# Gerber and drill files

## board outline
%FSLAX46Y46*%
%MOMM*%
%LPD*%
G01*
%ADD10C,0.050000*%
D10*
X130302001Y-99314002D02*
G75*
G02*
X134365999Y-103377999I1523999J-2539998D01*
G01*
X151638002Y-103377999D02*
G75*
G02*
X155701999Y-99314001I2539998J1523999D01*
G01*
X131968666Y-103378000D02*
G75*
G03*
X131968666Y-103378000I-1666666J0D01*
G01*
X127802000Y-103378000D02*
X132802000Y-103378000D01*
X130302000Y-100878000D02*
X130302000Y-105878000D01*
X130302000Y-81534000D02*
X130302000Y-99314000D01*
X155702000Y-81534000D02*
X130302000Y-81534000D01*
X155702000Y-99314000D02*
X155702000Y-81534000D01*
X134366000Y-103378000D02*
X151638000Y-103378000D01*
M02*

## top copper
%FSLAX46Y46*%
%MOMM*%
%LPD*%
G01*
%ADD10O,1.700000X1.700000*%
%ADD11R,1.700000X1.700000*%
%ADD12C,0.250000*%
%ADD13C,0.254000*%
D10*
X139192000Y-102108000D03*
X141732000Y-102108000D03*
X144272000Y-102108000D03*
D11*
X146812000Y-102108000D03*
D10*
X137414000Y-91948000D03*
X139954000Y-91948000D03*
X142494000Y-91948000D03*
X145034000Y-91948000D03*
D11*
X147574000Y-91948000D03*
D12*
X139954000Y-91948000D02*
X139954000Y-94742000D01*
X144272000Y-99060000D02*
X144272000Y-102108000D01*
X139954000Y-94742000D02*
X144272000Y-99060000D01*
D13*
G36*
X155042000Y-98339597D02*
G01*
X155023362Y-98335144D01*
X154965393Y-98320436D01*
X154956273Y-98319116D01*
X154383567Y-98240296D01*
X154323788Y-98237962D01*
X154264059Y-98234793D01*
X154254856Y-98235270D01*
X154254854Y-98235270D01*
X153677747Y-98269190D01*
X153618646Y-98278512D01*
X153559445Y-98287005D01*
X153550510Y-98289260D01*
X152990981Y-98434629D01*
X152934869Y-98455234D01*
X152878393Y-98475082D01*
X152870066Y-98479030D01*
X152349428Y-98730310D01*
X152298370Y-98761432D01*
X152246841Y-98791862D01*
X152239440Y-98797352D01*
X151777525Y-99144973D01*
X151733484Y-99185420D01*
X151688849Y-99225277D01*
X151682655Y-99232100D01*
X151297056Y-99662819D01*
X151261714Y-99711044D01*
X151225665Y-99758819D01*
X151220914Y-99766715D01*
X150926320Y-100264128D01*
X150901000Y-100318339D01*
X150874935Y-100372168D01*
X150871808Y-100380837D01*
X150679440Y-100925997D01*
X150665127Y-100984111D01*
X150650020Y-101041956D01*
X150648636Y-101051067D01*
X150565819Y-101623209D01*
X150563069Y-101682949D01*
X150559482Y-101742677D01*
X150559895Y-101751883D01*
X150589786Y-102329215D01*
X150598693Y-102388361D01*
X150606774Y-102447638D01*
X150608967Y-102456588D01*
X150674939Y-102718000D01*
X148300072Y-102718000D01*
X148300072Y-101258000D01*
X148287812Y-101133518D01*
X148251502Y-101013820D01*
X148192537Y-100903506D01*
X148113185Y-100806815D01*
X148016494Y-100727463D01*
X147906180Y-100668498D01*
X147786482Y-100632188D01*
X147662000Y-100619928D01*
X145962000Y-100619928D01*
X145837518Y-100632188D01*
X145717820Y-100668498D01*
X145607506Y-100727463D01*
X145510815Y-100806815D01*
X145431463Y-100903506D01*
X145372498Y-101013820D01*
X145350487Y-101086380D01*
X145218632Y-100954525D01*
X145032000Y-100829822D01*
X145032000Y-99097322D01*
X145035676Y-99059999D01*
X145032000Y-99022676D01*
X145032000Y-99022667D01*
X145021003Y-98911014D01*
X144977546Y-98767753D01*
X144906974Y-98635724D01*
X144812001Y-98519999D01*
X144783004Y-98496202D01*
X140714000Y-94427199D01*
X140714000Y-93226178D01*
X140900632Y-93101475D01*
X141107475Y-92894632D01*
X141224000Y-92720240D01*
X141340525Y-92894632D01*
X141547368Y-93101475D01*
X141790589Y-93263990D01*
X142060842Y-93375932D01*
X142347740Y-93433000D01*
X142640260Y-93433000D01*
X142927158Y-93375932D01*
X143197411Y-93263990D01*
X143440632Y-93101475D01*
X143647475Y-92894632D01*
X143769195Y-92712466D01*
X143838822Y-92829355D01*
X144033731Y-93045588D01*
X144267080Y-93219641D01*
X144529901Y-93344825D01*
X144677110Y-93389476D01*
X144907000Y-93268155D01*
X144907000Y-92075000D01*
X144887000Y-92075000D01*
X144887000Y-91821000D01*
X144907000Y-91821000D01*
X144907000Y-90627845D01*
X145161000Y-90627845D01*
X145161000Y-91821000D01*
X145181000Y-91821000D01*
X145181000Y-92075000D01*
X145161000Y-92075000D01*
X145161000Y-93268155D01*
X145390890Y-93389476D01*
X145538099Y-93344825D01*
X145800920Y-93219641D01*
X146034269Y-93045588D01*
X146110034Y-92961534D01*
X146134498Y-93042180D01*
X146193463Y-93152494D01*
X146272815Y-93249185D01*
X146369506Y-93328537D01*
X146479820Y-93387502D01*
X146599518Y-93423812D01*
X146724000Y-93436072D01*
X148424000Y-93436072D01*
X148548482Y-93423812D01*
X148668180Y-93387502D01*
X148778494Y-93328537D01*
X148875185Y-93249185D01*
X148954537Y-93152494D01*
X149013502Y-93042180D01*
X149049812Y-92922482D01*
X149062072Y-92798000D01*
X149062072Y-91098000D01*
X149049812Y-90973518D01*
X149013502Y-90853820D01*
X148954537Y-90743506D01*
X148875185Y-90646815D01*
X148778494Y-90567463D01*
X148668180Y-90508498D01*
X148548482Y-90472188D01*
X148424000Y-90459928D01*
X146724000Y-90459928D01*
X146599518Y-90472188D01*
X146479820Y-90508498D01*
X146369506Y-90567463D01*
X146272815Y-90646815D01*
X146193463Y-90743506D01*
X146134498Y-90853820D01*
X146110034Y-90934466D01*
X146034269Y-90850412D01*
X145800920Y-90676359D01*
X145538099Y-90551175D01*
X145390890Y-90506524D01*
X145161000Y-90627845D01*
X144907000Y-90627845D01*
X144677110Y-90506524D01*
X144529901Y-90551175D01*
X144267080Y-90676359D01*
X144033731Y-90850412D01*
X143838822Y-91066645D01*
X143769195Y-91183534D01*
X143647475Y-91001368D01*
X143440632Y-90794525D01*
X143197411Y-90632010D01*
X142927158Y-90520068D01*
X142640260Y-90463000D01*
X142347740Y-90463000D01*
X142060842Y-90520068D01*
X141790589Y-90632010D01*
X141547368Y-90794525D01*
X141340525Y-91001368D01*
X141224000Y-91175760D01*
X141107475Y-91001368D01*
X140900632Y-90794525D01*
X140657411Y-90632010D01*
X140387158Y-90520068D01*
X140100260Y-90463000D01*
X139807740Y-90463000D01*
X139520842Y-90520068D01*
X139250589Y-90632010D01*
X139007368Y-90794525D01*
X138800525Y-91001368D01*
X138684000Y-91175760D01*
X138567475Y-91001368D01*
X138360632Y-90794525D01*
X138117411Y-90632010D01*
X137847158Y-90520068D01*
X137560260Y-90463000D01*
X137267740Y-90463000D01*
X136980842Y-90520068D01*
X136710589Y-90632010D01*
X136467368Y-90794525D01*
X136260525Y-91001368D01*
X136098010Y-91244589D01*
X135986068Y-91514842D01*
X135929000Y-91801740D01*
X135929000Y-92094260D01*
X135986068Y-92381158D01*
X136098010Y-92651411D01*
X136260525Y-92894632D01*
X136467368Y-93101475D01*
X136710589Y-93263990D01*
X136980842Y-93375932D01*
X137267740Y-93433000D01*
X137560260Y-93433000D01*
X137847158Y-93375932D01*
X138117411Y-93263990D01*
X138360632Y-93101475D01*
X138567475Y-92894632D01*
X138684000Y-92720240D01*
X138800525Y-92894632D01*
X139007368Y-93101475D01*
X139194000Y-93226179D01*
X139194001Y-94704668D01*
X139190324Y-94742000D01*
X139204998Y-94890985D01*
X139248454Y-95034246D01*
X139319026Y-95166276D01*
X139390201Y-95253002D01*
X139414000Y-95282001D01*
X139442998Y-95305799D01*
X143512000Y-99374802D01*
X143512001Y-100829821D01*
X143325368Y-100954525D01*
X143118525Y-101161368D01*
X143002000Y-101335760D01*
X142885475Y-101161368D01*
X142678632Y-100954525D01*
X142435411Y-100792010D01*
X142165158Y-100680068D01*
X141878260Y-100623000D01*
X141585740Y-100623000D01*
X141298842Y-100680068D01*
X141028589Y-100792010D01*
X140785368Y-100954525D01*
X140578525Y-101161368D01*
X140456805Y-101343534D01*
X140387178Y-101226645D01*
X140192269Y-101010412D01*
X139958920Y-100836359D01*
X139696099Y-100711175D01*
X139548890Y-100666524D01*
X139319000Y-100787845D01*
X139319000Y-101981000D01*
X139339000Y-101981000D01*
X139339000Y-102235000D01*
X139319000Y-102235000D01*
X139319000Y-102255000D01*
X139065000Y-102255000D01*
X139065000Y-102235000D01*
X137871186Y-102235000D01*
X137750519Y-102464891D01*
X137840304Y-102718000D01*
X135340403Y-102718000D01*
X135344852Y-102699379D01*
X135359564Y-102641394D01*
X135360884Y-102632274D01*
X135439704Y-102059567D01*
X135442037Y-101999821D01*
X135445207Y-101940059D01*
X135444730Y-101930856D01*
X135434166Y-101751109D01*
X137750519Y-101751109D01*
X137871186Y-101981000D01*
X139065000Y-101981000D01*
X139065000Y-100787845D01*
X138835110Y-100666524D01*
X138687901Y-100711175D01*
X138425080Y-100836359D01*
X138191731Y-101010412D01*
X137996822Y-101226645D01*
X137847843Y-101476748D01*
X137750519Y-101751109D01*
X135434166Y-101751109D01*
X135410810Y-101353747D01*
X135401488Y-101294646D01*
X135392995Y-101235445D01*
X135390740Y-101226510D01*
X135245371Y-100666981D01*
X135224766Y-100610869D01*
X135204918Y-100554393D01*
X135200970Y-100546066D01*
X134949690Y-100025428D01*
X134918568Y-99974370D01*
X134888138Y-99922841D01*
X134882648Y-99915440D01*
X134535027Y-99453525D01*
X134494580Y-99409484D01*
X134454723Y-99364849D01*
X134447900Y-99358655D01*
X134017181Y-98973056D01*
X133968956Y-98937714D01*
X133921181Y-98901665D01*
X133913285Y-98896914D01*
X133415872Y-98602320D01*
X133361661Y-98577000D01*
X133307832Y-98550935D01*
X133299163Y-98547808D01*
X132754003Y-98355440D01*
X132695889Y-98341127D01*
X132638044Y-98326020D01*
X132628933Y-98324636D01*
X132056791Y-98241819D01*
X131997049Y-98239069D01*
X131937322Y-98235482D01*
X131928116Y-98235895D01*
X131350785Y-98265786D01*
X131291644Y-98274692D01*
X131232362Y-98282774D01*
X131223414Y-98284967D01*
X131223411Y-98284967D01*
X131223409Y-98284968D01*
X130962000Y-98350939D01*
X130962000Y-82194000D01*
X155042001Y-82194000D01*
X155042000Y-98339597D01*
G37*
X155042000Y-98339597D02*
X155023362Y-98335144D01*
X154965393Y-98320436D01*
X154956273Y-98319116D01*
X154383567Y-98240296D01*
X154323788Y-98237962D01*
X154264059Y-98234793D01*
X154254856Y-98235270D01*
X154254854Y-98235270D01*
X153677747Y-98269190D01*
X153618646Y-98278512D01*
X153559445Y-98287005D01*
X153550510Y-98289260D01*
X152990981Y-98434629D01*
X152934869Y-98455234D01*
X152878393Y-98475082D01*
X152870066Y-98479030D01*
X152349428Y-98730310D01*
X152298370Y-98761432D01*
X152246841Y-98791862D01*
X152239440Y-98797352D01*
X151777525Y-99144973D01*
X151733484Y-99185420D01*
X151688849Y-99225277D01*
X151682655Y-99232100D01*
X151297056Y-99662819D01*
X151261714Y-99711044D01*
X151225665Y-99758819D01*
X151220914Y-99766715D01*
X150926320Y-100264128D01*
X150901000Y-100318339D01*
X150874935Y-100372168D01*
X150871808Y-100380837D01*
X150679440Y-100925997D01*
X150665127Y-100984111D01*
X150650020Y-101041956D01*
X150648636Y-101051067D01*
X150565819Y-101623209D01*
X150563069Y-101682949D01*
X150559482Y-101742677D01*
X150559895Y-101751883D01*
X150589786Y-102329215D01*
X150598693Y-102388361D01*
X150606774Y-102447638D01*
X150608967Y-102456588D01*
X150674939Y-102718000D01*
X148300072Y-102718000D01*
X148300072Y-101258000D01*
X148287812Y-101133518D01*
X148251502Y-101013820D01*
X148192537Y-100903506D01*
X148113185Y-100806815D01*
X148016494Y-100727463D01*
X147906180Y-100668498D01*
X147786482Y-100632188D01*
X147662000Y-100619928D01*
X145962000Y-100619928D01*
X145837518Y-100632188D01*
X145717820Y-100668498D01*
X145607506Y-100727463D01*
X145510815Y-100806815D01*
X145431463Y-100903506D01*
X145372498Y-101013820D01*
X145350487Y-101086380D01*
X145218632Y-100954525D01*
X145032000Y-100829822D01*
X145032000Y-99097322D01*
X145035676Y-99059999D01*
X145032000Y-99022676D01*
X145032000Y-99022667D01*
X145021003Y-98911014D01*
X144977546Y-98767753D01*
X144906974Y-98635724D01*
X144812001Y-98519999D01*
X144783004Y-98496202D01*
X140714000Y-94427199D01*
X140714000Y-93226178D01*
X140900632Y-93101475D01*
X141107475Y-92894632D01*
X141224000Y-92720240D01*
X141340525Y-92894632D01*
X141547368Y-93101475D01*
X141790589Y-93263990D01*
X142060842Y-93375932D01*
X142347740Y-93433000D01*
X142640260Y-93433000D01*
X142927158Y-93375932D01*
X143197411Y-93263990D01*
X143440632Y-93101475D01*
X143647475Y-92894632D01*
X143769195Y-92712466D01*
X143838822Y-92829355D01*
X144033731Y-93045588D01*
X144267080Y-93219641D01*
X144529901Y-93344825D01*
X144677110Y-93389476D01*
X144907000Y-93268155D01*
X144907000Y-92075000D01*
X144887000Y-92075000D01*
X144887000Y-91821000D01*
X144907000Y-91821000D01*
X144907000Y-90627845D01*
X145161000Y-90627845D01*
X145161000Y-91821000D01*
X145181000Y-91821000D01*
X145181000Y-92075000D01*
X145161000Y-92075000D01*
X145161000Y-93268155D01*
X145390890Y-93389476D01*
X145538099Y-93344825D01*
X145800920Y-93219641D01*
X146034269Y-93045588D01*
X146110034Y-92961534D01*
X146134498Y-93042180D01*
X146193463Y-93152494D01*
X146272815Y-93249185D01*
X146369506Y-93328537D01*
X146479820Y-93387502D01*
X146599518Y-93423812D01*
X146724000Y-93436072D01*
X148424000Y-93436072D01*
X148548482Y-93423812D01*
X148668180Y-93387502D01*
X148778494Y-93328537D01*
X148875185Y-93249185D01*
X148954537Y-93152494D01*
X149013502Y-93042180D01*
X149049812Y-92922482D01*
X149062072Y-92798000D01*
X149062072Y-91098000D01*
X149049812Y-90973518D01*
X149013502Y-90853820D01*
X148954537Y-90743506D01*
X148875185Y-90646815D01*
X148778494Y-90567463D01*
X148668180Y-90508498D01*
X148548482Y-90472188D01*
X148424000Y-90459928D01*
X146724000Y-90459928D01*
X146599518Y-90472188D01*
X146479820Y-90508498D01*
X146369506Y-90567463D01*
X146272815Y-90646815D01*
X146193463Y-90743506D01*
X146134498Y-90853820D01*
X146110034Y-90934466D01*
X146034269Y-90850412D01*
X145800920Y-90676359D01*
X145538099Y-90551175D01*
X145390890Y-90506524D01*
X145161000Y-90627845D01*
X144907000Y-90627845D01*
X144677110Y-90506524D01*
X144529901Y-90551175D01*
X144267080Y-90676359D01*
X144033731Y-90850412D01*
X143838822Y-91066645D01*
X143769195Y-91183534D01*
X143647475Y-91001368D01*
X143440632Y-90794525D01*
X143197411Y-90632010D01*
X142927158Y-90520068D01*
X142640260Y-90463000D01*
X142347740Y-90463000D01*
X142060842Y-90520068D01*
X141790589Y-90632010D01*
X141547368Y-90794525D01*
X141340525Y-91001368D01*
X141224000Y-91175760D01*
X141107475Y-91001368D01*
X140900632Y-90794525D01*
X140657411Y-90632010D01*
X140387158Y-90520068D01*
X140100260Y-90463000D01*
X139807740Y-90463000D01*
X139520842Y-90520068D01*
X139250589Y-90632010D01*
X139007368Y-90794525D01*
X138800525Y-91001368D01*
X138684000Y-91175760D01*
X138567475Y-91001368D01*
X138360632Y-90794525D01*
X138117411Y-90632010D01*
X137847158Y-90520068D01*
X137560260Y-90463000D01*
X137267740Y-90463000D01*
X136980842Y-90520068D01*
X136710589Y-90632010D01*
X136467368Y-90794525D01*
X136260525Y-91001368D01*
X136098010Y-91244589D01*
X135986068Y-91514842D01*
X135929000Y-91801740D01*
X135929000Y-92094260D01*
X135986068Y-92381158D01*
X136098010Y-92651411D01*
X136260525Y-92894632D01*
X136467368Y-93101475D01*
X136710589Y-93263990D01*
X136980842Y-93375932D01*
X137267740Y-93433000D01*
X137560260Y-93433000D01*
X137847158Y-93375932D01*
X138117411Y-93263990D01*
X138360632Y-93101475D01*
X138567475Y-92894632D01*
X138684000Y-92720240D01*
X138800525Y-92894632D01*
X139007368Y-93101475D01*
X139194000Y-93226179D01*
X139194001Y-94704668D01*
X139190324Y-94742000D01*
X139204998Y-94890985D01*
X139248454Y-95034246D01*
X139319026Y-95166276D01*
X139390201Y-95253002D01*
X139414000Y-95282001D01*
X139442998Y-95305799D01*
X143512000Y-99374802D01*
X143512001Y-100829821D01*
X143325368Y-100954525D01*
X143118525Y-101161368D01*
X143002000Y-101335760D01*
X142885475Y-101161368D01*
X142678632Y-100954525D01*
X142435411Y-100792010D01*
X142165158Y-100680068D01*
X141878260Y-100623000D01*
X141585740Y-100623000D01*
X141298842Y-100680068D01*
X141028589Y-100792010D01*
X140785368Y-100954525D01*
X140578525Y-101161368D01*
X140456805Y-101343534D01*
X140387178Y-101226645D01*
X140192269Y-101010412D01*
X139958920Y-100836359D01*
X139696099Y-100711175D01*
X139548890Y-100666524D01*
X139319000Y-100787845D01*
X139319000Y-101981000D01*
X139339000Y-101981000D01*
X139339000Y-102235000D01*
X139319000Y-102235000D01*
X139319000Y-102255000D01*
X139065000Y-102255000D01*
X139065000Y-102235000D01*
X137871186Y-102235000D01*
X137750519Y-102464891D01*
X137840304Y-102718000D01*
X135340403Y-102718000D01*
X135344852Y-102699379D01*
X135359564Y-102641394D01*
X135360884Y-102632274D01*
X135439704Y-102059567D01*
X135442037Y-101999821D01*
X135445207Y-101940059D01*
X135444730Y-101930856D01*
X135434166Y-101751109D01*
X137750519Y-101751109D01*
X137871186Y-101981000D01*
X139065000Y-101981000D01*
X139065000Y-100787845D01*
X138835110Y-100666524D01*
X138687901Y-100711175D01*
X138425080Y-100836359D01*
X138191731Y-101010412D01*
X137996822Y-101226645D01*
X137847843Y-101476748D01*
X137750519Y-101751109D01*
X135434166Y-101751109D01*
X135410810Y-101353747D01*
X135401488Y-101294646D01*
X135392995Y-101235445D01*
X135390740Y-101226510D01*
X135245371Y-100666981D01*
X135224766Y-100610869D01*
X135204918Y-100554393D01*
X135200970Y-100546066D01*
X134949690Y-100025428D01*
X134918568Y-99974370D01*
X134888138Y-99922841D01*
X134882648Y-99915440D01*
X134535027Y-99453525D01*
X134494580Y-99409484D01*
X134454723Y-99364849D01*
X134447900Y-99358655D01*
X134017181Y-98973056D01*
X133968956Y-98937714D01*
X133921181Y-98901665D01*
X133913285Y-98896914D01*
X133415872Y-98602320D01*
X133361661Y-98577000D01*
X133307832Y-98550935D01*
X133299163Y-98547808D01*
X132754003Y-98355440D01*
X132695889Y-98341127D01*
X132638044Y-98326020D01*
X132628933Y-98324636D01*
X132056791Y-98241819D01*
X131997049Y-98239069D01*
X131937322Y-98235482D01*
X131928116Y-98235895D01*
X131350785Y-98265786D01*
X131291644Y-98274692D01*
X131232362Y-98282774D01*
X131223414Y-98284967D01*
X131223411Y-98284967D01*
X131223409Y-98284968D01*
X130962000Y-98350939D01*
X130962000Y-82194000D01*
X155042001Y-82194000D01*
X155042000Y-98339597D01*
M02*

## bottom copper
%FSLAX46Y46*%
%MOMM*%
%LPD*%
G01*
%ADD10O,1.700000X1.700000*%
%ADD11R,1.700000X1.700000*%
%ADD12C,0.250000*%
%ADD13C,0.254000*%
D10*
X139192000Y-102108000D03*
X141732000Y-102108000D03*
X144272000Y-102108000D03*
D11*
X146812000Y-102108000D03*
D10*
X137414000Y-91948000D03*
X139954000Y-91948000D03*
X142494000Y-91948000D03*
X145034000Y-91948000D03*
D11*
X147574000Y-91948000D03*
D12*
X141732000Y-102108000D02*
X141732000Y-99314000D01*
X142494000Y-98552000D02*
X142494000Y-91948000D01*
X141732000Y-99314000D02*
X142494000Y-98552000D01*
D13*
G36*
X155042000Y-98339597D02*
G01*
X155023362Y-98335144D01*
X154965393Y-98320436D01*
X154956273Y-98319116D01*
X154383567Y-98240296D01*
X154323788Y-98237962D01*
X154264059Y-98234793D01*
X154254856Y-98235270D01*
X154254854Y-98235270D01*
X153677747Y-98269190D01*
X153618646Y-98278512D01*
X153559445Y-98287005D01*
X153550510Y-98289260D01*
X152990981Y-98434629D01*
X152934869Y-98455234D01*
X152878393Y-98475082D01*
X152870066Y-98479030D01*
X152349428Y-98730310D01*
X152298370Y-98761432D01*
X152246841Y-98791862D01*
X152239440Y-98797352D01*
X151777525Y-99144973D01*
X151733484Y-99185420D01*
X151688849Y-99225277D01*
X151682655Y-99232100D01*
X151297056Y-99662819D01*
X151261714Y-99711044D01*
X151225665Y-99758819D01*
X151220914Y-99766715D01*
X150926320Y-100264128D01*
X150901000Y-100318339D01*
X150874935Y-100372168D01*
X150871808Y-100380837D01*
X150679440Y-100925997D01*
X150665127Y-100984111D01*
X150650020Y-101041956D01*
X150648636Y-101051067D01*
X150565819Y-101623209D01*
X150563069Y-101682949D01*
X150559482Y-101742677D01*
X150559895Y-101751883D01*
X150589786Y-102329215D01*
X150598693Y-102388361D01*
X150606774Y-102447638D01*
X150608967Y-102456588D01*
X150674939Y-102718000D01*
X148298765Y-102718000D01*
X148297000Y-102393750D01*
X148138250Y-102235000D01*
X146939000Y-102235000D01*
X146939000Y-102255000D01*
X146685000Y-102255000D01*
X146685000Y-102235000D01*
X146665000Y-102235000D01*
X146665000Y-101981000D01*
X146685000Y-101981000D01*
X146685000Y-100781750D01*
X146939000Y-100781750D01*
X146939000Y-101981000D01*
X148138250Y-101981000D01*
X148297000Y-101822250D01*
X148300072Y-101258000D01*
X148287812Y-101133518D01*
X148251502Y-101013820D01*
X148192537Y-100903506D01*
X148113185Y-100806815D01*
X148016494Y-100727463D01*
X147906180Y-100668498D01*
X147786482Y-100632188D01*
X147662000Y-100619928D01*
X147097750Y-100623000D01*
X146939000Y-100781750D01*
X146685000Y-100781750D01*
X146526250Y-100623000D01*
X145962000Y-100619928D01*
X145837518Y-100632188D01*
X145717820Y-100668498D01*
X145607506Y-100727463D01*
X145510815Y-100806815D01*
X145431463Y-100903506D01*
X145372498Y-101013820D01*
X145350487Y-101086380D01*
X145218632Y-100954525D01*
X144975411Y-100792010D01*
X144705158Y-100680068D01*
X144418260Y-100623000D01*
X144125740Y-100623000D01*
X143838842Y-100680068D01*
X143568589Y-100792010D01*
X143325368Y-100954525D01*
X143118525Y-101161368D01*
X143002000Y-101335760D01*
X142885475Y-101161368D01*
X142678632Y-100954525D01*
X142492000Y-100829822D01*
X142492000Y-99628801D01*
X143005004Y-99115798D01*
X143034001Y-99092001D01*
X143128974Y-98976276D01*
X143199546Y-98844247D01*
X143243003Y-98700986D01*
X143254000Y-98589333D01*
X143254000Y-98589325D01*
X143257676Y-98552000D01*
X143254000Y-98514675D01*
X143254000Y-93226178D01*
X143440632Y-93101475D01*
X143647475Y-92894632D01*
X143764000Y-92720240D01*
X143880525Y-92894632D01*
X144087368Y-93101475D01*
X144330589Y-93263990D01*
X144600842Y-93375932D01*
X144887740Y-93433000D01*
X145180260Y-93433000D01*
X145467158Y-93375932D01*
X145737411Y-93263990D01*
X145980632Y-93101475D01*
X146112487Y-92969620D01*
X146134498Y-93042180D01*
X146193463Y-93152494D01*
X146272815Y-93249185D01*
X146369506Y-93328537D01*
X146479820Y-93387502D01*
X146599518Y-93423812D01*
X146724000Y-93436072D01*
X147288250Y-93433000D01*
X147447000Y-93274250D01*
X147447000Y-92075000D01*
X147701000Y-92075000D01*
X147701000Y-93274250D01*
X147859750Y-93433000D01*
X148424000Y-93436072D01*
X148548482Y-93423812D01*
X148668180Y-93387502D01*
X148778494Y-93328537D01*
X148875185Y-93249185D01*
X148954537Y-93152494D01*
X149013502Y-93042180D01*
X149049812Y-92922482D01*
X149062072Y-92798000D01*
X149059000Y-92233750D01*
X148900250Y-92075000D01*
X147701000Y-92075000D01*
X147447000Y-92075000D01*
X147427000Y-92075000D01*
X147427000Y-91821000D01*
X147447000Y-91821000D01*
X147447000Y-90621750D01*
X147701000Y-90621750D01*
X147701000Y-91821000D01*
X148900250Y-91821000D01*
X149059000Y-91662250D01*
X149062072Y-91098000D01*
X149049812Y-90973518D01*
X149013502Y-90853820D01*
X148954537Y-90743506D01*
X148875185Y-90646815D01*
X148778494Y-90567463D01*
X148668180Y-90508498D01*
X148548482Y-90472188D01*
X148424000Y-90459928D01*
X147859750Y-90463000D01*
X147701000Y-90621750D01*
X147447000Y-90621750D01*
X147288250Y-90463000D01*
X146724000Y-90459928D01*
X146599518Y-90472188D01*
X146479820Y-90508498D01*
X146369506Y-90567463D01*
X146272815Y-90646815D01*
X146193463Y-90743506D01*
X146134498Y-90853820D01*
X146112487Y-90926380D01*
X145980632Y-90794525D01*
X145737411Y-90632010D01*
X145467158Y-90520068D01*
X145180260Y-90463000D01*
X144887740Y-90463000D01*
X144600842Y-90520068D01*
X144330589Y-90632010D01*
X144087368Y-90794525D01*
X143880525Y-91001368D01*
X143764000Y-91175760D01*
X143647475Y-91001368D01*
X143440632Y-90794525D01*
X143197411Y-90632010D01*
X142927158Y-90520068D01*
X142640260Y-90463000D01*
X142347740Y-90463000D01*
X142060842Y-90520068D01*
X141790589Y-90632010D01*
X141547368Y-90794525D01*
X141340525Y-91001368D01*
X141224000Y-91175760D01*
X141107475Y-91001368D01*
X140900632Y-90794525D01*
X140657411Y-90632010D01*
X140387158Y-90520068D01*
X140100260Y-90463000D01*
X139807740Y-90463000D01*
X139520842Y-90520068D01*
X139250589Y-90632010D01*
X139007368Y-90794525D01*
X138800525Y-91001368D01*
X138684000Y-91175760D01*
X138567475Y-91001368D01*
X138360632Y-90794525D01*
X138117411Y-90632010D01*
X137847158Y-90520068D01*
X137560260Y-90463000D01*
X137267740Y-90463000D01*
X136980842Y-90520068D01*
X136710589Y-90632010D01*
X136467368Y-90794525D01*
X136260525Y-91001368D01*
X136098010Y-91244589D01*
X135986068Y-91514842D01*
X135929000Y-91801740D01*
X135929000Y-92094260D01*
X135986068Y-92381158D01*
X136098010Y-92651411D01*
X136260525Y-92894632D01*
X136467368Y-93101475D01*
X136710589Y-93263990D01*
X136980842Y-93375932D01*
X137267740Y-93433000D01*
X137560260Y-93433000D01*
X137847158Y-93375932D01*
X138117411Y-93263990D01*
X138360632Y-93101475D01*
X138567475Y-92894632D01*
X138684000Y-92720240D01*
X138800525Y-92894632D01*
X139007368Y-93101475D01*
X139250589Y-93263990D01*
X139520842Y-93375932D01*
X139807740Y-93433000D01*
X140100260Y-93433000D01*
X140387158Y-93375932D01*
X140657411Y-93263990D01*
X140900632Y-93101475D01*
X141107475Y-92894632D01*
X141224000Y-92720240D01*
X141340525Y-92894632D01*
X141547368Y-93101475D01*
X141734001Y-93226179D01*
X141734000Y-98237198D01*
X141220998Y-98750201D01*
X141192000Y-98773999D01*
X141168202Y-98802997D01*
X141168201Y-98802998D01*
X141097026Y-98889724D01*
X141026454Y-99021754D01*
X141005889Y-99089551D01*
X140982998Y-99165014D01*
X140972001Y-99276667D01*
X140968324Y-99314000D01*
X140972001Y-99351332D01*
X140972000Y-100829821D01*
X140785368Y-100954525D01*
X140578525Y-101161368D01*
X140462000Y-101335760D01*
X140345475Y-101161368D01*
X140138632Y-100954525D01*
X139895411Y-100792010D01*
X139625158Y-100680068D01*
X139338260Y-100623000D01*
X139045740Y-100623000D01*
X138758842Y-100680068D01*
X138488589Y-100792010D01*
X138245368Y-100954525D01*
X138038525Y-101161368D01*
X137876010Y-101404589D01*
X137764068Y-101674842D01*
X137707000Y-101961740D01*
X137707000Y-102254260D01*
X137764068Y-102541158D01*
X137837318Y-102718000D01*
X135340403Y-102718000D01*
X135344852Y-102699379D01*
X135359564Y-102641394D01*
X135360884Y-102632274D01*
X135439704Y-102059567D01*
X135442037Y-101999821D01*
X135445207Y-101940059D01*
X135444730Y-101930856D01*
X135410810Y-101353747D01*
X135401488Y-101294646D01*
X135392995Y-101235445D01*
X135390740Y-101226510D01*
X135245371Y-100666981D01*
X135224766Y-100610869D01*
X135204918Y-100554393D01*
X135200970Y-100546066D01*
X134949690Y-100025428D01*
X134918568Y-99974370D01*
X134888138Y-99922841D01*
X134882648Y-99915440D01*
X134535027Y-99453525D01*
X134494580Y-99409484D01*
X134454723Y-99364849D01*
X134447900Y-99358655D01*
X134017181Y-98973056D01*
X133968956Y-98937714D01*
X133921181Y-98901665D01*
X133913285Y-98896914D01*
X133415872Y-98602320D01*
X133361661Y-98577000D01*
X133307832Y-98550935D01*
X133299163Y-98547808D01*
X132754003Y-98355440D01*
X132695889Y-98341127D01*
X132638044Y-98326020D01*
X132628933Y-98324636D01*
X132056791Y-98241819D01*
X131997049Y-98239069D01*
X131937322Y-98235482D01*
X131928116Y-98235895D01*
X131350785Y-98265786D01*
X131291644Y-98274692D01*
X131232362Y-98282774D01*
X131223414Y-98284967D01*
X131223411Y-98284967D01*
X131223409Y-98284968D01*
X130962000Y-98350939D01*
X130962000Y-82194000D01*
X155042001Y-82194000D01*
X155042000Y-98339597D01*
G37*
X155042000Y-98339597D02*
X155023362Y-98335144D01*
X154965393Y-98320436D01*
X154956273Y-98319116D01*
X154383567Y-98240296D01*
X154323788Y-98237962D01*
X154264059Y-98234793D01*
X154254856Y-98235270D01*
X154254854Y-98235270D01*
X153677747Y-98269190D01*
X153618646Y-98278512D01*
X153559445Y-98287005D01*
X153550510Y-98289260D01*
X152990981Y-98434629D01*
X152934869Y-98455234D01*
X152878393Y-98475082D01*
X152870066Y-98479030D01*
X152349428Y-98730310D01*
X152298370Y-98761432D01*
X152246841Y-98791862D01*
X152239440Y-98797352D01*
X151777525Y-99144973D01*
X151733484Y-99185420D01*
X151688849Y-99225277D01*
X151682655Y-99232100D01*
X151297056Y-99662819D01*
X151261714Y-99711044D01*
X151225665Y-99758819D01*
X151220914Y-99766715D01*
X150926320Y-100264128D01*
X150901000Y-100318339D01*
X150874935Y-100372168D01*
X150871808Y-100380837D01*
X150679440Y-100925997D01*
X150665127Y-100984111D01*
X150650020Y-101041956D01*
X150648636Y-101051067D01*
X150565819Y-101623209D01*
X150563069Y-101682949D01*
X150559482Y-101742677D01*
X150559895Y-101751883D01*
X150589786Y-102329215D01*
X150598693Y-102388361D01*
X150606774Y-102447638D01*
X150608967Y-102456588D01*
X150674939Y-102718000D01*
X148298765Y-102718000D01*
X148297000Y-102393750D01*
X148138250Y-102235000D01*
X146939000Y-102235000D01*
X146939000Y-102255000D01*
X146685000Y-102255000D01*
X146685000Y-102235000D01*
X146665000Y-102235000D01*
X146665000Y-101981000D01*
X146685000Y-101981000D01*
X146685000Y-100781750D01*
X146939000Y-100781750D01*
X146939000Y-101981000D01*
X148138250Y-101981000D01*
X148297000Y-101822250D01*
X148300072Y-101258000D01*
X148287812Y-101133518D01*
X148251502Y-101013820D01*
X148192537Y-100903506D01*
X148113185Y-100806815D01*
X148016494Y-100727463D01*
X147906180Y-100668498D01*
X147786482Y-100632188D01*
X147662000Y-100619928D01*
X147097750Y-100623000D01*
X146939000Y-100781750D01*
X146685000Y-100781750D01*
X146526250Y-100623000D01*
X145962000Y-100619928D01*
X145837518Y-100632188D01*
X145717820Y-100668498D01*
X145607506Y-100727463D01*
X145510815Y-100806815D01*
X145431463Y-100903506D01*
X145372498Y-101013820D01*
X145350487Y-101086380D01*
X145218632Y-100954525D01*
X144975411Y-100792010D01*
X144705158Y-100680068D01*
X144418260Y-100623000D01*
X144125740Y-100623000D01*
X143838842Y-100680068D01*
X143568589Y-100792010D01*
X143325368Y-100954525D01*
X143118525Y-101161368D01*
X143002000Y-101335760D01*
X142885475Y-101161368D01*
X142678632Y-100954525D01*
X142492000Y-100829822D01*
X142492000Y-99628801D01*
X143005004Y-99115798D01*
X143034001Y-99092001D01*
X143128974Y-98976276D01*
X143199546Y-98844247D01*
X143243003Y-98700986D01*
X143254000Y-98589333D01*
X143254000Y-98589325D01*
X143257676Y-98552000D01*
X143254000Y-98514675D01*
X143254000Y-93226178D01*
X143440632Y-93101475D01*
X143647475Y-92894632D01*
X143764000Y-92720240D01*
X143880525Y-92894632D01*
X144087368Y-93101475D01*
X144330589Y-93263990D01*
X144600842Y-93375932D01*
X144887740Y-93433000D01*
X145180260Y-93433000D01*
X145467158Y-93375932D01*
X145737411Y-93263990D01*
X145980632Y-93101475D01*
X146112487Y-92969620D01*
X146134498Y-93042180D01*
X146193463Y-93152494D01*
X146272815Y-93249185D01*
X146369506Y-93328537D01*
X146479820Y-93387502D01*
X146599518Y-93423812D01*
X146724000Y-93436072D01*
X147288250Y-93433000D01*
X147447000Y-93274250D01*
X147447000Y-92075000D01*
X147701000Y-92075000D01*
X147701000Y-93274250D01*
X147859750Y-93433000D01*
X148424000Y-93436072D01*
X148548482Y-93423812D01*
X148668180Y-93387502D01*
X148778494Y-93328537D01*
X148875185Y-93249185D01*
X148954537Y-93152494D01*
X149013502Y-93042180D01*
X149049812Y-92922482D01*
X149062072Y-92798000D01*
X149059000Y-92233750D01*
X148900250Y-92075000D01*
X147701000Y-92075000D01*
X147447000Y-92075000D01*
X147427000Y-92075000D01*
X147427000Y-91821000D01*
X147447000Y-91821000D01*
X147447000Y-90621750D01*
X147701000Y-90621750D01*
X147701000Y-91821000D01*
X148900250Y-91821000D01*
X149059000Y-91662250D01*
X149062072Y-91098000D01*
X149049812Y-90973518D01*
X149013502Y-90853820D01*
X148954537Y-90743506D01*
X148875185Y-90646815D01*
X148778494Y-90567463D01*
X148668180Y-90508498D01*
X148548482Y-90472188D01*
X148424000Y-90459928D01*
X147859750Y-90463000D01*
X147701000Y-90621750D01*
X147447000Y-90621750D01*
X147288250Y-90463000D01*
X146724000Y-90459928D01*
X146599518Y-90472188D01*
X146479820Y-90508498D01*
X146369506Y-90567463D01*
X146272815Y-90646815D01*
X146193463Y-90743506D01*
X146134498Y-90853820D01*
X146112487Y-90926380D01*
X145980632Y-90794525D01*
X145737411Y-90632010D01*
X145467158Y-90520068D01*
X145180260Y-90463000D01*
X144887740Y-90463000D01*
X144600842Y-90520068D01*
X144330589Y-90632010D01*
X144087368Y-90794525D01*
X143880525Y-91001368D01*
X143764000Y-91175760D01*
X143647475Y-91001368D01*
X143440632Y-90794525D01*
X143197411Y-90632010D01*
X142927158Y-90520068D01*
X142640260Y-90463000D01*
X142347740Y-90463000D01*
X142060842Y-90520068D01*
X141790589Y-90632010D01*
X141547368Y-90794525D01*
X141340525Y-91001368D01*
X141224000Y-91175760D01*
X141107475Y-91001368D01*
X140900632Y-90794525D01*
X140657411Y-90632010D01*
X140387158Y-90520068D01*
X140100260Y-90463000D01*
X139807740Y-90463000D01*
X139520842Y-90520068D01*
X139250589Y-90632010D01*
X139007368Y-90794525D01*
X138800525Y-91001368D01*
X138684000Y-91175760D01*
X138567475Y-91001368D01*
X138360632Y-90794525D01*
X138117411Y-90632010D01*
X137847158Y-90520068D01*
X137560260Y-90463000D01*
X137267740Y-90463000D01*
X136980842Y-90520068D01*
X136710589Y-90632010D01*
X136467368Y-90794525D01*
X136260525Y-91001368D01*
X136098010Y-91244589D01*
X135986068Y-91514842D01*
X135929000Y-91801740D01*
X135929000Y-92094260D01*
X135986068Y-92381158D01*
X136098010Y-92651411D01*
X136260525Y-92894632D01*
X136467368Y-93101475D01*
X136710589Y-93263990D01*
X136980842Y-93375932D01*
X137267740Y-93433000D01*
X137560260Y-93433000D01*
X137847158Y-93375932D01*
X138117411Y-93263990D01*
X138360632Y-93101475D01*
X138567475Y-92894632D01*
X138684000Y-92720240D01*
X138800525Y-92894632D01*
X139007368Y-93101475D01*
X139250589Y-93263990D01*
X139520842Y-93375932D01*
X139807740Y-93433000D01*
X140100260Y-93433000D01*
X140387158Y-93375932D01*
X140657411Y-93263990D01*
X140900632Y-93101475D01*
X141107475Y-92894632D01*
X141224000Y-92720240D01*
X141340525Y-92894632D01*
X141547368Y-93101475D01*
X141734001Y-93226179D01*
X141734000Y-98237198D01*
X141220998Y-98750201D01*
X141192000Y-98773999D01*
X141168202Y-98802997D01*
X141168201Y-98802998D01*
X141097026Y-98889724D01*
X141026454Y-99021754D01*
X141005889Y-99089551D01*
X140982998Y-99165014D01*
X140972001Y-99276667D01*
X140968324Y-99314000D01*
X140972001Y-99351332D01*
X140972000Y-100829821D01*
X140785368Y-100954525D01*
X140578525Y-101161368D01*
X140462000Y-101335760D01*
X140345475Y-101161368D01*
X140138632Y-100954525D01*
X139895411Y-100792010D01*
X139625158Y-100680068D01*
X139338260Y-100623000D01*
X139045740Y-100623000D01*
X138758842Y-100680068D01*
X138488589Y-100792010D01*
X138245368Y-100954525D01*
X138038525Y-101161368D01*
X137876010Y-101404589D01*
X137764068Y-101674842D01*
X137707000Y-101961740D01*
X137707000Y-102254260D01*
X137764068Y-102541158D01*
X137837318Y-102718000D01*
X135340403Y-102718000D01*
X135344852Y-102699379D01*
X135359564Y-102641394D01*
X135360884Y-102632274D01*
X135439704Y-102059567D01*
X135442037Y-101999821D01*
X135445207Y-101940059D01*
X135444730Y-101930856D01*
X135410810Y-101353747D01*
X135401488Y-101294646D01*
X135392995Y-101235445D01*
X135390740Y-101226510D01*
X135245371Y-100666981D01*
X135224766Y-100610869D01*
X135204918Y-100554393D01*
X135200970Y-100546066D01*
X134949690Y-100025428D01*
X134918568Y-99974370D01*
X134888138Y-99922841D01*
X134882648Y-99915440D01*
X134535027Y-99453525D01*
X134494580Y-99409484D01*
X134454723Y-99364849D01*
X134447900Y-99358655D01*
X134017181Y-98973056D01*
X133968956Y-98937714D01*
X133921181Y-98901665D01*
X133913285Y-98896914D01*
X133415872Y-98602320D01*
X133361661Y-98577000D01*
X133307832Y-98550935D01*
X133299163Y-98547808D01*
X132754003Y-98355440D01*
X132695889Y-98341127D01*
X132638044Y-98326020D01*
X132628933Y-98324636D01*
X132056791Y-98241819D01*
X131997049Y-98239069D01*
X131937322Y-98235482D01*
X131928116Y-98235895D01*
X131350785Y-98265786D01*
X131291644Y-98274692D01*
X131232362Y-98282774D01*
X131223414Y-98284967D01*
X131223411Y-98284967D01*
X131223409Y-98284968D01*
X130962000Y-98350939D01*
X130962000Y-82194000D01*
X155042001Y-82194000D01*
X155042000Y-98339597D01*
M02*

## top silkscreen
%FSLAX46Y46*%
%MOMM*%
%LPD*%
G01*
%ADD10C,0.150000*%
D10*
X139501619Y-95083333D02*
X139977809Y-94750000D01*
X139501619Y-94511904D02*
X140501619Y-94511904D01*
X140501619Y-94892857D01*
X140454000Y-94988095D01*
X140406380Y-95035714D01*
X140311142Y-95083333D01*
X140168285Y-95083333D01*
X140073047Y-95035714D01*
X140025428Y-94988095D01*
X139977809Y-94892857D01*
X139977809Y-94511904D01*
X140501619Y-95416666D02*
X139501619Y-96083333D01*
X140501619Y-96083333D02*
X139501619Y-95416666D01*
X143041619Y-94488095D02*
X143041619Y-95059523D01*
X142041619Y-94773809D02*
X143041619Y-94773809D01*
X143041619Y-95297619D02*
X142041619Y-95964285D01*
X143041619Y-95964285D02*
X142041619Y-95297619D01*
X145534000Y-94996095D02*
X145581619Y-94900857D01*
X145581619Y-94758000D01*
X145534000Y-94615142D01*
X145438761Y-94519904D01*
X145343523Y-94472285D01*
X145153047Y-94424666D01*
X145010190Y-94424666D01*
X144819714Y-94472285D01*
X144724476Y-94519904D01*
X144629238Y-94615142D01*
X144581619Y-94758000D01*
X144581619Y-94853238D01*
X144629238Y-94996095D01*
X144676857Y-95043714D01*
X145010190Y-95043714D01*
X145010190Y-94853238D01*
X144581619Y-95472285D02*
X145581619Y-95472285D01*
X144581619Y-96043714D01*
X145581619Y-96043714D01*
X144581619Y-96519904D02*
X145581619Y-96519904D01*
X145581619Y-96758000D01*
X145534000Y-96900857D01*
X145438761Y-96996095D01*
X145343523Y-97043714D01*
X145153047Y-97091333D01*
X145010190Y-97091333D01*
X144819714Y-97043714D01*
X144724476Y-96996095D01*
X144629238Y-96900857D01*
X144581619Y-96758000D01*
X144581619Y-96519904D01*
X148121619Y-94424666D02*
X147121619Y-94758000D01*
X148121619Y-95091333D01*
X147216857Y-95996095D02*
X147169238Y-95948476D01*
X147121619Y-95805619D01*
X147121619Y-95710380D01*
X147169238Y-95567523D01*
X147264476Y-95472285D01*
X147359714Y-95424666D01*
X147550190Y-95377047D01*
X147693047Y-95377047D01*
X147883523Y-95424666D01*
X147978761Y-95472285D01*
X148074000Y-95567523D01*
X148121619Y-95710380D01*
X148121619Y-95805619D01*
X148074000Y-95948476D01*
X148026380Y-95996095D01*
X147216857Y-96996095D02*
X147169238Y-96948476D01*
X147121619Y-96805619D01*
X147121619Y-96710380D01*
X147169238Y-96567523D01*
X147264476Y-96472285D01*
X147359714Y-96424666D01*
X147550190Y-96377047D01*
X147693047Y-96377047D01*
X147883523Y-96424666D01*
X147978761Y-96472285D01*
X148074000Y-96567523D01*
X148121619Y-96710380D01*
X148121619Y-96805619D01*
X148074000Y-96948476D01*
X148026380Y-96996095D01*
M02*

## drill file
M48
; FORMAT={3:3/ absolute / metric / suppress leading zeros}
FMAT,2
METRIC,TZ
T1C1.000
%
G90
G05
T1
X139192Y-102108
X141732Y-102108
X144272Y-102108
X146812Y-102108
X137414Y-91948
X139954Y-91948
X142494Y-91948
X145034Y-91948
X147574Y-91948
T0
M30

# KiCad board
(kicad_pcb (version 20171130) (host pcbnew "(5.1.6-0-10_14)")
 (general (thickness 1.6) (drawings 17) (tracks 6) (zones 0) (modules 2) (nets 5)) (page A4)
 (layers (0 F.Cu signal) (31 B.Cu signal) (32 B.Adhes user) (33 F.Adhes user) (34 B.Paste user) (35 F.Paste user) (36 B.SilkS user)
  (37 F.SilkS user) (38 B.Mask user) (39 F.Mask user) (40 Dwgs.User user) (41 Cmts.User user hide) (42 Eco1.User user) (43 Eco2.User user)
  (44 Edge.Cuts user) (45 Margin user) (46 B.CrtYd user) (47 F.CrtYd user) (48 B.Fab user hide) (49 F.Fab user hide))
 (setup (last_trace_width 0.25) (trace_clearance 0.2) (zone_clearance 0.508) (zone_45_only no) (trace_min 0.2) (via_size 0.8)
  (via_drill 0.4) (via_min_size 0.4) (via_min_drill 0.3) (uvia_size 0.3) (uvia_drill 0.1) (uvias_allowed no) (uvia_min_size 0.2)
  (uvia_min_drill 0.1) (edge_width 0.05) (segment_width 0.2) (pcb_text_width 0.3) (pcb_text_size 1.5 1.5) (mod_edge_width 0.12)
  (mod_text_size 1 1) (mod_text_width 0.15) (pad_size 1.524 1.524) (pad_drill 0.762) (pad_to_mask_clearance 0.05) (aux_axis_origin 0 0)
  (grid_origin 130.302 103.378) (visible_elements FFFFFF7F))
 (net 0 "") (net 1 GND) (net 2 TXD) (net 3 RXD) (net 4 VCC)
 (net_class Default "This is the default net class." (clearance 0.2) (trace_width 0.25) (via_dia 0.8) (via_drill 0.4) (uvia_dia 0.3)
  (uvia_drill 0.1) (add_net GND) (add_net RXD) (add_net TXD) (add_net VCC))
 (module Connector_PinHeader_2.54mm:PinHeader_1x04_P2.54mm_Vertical (layer B.Cu) (at 146.812 102.108 90)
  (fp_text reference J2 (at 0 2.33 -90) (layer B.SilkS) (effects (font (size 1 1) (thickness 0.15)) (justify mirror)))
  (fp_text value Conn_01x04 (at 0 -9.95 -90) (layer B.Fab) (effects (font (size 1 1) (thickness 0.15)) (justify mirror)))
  (pad 4 thru_hole oval (at 0 -7.62 90) (size 1.7 1.7) (drill 1) (layers *.Cu *.Mask) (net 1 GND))
  (pad 3 thru_hole oval (at 0 -5.08 90) (size 1.7 1.7) (drill 1) (layers *.Cu *.Mask) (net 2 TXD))
  (pad 2 thru_hole oval (at 0 -2.54 90) (size 1.7 1.7) (drill 1) (layers *.Cu *.Mask) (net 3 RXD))
  (pad 1 thru_hole rect (at 0 0 90) (size 1.7 1.7) (drill 1) (layers *.Cu *.Mask) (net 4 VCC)))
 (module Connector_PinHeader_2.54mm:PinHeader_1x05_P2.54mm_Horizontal (layer B.Cu) (at 147.574 91.948 90)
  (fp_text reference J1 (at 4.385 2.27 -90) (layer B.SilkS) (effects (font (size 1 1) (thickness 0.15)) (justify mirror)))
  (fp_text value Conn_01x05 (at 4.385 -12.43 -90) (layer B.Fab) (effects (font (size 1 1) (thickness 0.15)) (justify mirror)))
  (pad 5 thru_hole oval (at 0 -10.16 90) (size 1.7 1.7) (drill 1) (layers *.Cu *.Mask))
  (pad 4 thru_hole oval (at 0 -7.62 90) (size 1.7 1.7) (drill 1) (layers *.Cu *.Mask) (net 3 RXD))
  (pad 3 thru_hole oval (at 0 -5.08 90) (size 1.7 1.7) (drill 1) (layers *.Cu *.Mask) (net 2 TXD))
  (pad 2 thru_hole oval (at 0 -2.54 90) (size 1.7 1.7) (drill 1) (layers *.Cu *.Mask) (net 1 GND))
  (pad 1 thru_hole rect (at 0 0 90) (size 1.7 1.7) (drill 1) (layers *.Cu *.Mask) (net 4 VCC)))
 (gr_arc (start 131.826 101.854) (end 134.365999 103.377999) (angle -151.9275131) (layer Edge.Cuts) (width 0.05))
 (gr_arc (start 154.178 101.854) (end 155.701999 99.314001) (angle -151.9275131) (layer Edge.Cuts) (width 0.05))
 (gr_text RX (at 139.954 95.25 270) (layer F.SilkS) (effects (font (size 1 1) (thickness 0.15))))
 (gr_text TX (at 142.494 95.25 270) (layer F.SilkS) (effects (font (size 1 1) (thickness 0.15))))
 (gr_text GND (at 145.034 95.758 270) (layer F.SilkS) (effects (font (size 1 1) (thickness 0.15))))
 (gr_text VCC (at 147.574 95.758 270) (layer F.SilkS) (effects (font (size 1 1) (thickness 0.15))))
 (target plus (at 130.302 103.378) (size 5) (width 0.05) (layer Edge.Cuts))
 (gr_line (start 130.302 81.534) (end 130.302 99.314) (layer Edge.Cuts) (width 0.05))
 (gr_line (start 155.702 81.534) (end 130.302 81.534) (layer Edge.Cuts) (width 0.05))
 (gr_line (start 155.702 99.314) (end 155.702 81.534) (layer Edge.Cuts) (width 0.05))
 (gr_line (start 134.366 103.378) (end 151.638 103.378) (layer Edge.Cuts) (width 0.05))
 (segment (start 139.954 91.948) (end 139.954 94.742) (width 0.25) (layer F.Cu) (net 3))
 (segment (start 144.272 99.06) (end 144.272 102.108) (width 0.25) (layer F.Cu) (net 3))
 (segment (start 139.954 94.742) (end 144.272 99.06) (width 0.25) (layer F.Cu) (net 3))
 (segment (start 141.732 102.108) (end 141.732 99.314) (width 0.25) (layer B.Cu) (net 2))
 (segment (start 142.494 98.552) (end 142.494 91.948) (width 0.25) (layer B.Cu) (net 2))
 (segment (start 141.732 99.314) (end 142.494 98.552) (width 0.25) (layer B.Cu) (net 2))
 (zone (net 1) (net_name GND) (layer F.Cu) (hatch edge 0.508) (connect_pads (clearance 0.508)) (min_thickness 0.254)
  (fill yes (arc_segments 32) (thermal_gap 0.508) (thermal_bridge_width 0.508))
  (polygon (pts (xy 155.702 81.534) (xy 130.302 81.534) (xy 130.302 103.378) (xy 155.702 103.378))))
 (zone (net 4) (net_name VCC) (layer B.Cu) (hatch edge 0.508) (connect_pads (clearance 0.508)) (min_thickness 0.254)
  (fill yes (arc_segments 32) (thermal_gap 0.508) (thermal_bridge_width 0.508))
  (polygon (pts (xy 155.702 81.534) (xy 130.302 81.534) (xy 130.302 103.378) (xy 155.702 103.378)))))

